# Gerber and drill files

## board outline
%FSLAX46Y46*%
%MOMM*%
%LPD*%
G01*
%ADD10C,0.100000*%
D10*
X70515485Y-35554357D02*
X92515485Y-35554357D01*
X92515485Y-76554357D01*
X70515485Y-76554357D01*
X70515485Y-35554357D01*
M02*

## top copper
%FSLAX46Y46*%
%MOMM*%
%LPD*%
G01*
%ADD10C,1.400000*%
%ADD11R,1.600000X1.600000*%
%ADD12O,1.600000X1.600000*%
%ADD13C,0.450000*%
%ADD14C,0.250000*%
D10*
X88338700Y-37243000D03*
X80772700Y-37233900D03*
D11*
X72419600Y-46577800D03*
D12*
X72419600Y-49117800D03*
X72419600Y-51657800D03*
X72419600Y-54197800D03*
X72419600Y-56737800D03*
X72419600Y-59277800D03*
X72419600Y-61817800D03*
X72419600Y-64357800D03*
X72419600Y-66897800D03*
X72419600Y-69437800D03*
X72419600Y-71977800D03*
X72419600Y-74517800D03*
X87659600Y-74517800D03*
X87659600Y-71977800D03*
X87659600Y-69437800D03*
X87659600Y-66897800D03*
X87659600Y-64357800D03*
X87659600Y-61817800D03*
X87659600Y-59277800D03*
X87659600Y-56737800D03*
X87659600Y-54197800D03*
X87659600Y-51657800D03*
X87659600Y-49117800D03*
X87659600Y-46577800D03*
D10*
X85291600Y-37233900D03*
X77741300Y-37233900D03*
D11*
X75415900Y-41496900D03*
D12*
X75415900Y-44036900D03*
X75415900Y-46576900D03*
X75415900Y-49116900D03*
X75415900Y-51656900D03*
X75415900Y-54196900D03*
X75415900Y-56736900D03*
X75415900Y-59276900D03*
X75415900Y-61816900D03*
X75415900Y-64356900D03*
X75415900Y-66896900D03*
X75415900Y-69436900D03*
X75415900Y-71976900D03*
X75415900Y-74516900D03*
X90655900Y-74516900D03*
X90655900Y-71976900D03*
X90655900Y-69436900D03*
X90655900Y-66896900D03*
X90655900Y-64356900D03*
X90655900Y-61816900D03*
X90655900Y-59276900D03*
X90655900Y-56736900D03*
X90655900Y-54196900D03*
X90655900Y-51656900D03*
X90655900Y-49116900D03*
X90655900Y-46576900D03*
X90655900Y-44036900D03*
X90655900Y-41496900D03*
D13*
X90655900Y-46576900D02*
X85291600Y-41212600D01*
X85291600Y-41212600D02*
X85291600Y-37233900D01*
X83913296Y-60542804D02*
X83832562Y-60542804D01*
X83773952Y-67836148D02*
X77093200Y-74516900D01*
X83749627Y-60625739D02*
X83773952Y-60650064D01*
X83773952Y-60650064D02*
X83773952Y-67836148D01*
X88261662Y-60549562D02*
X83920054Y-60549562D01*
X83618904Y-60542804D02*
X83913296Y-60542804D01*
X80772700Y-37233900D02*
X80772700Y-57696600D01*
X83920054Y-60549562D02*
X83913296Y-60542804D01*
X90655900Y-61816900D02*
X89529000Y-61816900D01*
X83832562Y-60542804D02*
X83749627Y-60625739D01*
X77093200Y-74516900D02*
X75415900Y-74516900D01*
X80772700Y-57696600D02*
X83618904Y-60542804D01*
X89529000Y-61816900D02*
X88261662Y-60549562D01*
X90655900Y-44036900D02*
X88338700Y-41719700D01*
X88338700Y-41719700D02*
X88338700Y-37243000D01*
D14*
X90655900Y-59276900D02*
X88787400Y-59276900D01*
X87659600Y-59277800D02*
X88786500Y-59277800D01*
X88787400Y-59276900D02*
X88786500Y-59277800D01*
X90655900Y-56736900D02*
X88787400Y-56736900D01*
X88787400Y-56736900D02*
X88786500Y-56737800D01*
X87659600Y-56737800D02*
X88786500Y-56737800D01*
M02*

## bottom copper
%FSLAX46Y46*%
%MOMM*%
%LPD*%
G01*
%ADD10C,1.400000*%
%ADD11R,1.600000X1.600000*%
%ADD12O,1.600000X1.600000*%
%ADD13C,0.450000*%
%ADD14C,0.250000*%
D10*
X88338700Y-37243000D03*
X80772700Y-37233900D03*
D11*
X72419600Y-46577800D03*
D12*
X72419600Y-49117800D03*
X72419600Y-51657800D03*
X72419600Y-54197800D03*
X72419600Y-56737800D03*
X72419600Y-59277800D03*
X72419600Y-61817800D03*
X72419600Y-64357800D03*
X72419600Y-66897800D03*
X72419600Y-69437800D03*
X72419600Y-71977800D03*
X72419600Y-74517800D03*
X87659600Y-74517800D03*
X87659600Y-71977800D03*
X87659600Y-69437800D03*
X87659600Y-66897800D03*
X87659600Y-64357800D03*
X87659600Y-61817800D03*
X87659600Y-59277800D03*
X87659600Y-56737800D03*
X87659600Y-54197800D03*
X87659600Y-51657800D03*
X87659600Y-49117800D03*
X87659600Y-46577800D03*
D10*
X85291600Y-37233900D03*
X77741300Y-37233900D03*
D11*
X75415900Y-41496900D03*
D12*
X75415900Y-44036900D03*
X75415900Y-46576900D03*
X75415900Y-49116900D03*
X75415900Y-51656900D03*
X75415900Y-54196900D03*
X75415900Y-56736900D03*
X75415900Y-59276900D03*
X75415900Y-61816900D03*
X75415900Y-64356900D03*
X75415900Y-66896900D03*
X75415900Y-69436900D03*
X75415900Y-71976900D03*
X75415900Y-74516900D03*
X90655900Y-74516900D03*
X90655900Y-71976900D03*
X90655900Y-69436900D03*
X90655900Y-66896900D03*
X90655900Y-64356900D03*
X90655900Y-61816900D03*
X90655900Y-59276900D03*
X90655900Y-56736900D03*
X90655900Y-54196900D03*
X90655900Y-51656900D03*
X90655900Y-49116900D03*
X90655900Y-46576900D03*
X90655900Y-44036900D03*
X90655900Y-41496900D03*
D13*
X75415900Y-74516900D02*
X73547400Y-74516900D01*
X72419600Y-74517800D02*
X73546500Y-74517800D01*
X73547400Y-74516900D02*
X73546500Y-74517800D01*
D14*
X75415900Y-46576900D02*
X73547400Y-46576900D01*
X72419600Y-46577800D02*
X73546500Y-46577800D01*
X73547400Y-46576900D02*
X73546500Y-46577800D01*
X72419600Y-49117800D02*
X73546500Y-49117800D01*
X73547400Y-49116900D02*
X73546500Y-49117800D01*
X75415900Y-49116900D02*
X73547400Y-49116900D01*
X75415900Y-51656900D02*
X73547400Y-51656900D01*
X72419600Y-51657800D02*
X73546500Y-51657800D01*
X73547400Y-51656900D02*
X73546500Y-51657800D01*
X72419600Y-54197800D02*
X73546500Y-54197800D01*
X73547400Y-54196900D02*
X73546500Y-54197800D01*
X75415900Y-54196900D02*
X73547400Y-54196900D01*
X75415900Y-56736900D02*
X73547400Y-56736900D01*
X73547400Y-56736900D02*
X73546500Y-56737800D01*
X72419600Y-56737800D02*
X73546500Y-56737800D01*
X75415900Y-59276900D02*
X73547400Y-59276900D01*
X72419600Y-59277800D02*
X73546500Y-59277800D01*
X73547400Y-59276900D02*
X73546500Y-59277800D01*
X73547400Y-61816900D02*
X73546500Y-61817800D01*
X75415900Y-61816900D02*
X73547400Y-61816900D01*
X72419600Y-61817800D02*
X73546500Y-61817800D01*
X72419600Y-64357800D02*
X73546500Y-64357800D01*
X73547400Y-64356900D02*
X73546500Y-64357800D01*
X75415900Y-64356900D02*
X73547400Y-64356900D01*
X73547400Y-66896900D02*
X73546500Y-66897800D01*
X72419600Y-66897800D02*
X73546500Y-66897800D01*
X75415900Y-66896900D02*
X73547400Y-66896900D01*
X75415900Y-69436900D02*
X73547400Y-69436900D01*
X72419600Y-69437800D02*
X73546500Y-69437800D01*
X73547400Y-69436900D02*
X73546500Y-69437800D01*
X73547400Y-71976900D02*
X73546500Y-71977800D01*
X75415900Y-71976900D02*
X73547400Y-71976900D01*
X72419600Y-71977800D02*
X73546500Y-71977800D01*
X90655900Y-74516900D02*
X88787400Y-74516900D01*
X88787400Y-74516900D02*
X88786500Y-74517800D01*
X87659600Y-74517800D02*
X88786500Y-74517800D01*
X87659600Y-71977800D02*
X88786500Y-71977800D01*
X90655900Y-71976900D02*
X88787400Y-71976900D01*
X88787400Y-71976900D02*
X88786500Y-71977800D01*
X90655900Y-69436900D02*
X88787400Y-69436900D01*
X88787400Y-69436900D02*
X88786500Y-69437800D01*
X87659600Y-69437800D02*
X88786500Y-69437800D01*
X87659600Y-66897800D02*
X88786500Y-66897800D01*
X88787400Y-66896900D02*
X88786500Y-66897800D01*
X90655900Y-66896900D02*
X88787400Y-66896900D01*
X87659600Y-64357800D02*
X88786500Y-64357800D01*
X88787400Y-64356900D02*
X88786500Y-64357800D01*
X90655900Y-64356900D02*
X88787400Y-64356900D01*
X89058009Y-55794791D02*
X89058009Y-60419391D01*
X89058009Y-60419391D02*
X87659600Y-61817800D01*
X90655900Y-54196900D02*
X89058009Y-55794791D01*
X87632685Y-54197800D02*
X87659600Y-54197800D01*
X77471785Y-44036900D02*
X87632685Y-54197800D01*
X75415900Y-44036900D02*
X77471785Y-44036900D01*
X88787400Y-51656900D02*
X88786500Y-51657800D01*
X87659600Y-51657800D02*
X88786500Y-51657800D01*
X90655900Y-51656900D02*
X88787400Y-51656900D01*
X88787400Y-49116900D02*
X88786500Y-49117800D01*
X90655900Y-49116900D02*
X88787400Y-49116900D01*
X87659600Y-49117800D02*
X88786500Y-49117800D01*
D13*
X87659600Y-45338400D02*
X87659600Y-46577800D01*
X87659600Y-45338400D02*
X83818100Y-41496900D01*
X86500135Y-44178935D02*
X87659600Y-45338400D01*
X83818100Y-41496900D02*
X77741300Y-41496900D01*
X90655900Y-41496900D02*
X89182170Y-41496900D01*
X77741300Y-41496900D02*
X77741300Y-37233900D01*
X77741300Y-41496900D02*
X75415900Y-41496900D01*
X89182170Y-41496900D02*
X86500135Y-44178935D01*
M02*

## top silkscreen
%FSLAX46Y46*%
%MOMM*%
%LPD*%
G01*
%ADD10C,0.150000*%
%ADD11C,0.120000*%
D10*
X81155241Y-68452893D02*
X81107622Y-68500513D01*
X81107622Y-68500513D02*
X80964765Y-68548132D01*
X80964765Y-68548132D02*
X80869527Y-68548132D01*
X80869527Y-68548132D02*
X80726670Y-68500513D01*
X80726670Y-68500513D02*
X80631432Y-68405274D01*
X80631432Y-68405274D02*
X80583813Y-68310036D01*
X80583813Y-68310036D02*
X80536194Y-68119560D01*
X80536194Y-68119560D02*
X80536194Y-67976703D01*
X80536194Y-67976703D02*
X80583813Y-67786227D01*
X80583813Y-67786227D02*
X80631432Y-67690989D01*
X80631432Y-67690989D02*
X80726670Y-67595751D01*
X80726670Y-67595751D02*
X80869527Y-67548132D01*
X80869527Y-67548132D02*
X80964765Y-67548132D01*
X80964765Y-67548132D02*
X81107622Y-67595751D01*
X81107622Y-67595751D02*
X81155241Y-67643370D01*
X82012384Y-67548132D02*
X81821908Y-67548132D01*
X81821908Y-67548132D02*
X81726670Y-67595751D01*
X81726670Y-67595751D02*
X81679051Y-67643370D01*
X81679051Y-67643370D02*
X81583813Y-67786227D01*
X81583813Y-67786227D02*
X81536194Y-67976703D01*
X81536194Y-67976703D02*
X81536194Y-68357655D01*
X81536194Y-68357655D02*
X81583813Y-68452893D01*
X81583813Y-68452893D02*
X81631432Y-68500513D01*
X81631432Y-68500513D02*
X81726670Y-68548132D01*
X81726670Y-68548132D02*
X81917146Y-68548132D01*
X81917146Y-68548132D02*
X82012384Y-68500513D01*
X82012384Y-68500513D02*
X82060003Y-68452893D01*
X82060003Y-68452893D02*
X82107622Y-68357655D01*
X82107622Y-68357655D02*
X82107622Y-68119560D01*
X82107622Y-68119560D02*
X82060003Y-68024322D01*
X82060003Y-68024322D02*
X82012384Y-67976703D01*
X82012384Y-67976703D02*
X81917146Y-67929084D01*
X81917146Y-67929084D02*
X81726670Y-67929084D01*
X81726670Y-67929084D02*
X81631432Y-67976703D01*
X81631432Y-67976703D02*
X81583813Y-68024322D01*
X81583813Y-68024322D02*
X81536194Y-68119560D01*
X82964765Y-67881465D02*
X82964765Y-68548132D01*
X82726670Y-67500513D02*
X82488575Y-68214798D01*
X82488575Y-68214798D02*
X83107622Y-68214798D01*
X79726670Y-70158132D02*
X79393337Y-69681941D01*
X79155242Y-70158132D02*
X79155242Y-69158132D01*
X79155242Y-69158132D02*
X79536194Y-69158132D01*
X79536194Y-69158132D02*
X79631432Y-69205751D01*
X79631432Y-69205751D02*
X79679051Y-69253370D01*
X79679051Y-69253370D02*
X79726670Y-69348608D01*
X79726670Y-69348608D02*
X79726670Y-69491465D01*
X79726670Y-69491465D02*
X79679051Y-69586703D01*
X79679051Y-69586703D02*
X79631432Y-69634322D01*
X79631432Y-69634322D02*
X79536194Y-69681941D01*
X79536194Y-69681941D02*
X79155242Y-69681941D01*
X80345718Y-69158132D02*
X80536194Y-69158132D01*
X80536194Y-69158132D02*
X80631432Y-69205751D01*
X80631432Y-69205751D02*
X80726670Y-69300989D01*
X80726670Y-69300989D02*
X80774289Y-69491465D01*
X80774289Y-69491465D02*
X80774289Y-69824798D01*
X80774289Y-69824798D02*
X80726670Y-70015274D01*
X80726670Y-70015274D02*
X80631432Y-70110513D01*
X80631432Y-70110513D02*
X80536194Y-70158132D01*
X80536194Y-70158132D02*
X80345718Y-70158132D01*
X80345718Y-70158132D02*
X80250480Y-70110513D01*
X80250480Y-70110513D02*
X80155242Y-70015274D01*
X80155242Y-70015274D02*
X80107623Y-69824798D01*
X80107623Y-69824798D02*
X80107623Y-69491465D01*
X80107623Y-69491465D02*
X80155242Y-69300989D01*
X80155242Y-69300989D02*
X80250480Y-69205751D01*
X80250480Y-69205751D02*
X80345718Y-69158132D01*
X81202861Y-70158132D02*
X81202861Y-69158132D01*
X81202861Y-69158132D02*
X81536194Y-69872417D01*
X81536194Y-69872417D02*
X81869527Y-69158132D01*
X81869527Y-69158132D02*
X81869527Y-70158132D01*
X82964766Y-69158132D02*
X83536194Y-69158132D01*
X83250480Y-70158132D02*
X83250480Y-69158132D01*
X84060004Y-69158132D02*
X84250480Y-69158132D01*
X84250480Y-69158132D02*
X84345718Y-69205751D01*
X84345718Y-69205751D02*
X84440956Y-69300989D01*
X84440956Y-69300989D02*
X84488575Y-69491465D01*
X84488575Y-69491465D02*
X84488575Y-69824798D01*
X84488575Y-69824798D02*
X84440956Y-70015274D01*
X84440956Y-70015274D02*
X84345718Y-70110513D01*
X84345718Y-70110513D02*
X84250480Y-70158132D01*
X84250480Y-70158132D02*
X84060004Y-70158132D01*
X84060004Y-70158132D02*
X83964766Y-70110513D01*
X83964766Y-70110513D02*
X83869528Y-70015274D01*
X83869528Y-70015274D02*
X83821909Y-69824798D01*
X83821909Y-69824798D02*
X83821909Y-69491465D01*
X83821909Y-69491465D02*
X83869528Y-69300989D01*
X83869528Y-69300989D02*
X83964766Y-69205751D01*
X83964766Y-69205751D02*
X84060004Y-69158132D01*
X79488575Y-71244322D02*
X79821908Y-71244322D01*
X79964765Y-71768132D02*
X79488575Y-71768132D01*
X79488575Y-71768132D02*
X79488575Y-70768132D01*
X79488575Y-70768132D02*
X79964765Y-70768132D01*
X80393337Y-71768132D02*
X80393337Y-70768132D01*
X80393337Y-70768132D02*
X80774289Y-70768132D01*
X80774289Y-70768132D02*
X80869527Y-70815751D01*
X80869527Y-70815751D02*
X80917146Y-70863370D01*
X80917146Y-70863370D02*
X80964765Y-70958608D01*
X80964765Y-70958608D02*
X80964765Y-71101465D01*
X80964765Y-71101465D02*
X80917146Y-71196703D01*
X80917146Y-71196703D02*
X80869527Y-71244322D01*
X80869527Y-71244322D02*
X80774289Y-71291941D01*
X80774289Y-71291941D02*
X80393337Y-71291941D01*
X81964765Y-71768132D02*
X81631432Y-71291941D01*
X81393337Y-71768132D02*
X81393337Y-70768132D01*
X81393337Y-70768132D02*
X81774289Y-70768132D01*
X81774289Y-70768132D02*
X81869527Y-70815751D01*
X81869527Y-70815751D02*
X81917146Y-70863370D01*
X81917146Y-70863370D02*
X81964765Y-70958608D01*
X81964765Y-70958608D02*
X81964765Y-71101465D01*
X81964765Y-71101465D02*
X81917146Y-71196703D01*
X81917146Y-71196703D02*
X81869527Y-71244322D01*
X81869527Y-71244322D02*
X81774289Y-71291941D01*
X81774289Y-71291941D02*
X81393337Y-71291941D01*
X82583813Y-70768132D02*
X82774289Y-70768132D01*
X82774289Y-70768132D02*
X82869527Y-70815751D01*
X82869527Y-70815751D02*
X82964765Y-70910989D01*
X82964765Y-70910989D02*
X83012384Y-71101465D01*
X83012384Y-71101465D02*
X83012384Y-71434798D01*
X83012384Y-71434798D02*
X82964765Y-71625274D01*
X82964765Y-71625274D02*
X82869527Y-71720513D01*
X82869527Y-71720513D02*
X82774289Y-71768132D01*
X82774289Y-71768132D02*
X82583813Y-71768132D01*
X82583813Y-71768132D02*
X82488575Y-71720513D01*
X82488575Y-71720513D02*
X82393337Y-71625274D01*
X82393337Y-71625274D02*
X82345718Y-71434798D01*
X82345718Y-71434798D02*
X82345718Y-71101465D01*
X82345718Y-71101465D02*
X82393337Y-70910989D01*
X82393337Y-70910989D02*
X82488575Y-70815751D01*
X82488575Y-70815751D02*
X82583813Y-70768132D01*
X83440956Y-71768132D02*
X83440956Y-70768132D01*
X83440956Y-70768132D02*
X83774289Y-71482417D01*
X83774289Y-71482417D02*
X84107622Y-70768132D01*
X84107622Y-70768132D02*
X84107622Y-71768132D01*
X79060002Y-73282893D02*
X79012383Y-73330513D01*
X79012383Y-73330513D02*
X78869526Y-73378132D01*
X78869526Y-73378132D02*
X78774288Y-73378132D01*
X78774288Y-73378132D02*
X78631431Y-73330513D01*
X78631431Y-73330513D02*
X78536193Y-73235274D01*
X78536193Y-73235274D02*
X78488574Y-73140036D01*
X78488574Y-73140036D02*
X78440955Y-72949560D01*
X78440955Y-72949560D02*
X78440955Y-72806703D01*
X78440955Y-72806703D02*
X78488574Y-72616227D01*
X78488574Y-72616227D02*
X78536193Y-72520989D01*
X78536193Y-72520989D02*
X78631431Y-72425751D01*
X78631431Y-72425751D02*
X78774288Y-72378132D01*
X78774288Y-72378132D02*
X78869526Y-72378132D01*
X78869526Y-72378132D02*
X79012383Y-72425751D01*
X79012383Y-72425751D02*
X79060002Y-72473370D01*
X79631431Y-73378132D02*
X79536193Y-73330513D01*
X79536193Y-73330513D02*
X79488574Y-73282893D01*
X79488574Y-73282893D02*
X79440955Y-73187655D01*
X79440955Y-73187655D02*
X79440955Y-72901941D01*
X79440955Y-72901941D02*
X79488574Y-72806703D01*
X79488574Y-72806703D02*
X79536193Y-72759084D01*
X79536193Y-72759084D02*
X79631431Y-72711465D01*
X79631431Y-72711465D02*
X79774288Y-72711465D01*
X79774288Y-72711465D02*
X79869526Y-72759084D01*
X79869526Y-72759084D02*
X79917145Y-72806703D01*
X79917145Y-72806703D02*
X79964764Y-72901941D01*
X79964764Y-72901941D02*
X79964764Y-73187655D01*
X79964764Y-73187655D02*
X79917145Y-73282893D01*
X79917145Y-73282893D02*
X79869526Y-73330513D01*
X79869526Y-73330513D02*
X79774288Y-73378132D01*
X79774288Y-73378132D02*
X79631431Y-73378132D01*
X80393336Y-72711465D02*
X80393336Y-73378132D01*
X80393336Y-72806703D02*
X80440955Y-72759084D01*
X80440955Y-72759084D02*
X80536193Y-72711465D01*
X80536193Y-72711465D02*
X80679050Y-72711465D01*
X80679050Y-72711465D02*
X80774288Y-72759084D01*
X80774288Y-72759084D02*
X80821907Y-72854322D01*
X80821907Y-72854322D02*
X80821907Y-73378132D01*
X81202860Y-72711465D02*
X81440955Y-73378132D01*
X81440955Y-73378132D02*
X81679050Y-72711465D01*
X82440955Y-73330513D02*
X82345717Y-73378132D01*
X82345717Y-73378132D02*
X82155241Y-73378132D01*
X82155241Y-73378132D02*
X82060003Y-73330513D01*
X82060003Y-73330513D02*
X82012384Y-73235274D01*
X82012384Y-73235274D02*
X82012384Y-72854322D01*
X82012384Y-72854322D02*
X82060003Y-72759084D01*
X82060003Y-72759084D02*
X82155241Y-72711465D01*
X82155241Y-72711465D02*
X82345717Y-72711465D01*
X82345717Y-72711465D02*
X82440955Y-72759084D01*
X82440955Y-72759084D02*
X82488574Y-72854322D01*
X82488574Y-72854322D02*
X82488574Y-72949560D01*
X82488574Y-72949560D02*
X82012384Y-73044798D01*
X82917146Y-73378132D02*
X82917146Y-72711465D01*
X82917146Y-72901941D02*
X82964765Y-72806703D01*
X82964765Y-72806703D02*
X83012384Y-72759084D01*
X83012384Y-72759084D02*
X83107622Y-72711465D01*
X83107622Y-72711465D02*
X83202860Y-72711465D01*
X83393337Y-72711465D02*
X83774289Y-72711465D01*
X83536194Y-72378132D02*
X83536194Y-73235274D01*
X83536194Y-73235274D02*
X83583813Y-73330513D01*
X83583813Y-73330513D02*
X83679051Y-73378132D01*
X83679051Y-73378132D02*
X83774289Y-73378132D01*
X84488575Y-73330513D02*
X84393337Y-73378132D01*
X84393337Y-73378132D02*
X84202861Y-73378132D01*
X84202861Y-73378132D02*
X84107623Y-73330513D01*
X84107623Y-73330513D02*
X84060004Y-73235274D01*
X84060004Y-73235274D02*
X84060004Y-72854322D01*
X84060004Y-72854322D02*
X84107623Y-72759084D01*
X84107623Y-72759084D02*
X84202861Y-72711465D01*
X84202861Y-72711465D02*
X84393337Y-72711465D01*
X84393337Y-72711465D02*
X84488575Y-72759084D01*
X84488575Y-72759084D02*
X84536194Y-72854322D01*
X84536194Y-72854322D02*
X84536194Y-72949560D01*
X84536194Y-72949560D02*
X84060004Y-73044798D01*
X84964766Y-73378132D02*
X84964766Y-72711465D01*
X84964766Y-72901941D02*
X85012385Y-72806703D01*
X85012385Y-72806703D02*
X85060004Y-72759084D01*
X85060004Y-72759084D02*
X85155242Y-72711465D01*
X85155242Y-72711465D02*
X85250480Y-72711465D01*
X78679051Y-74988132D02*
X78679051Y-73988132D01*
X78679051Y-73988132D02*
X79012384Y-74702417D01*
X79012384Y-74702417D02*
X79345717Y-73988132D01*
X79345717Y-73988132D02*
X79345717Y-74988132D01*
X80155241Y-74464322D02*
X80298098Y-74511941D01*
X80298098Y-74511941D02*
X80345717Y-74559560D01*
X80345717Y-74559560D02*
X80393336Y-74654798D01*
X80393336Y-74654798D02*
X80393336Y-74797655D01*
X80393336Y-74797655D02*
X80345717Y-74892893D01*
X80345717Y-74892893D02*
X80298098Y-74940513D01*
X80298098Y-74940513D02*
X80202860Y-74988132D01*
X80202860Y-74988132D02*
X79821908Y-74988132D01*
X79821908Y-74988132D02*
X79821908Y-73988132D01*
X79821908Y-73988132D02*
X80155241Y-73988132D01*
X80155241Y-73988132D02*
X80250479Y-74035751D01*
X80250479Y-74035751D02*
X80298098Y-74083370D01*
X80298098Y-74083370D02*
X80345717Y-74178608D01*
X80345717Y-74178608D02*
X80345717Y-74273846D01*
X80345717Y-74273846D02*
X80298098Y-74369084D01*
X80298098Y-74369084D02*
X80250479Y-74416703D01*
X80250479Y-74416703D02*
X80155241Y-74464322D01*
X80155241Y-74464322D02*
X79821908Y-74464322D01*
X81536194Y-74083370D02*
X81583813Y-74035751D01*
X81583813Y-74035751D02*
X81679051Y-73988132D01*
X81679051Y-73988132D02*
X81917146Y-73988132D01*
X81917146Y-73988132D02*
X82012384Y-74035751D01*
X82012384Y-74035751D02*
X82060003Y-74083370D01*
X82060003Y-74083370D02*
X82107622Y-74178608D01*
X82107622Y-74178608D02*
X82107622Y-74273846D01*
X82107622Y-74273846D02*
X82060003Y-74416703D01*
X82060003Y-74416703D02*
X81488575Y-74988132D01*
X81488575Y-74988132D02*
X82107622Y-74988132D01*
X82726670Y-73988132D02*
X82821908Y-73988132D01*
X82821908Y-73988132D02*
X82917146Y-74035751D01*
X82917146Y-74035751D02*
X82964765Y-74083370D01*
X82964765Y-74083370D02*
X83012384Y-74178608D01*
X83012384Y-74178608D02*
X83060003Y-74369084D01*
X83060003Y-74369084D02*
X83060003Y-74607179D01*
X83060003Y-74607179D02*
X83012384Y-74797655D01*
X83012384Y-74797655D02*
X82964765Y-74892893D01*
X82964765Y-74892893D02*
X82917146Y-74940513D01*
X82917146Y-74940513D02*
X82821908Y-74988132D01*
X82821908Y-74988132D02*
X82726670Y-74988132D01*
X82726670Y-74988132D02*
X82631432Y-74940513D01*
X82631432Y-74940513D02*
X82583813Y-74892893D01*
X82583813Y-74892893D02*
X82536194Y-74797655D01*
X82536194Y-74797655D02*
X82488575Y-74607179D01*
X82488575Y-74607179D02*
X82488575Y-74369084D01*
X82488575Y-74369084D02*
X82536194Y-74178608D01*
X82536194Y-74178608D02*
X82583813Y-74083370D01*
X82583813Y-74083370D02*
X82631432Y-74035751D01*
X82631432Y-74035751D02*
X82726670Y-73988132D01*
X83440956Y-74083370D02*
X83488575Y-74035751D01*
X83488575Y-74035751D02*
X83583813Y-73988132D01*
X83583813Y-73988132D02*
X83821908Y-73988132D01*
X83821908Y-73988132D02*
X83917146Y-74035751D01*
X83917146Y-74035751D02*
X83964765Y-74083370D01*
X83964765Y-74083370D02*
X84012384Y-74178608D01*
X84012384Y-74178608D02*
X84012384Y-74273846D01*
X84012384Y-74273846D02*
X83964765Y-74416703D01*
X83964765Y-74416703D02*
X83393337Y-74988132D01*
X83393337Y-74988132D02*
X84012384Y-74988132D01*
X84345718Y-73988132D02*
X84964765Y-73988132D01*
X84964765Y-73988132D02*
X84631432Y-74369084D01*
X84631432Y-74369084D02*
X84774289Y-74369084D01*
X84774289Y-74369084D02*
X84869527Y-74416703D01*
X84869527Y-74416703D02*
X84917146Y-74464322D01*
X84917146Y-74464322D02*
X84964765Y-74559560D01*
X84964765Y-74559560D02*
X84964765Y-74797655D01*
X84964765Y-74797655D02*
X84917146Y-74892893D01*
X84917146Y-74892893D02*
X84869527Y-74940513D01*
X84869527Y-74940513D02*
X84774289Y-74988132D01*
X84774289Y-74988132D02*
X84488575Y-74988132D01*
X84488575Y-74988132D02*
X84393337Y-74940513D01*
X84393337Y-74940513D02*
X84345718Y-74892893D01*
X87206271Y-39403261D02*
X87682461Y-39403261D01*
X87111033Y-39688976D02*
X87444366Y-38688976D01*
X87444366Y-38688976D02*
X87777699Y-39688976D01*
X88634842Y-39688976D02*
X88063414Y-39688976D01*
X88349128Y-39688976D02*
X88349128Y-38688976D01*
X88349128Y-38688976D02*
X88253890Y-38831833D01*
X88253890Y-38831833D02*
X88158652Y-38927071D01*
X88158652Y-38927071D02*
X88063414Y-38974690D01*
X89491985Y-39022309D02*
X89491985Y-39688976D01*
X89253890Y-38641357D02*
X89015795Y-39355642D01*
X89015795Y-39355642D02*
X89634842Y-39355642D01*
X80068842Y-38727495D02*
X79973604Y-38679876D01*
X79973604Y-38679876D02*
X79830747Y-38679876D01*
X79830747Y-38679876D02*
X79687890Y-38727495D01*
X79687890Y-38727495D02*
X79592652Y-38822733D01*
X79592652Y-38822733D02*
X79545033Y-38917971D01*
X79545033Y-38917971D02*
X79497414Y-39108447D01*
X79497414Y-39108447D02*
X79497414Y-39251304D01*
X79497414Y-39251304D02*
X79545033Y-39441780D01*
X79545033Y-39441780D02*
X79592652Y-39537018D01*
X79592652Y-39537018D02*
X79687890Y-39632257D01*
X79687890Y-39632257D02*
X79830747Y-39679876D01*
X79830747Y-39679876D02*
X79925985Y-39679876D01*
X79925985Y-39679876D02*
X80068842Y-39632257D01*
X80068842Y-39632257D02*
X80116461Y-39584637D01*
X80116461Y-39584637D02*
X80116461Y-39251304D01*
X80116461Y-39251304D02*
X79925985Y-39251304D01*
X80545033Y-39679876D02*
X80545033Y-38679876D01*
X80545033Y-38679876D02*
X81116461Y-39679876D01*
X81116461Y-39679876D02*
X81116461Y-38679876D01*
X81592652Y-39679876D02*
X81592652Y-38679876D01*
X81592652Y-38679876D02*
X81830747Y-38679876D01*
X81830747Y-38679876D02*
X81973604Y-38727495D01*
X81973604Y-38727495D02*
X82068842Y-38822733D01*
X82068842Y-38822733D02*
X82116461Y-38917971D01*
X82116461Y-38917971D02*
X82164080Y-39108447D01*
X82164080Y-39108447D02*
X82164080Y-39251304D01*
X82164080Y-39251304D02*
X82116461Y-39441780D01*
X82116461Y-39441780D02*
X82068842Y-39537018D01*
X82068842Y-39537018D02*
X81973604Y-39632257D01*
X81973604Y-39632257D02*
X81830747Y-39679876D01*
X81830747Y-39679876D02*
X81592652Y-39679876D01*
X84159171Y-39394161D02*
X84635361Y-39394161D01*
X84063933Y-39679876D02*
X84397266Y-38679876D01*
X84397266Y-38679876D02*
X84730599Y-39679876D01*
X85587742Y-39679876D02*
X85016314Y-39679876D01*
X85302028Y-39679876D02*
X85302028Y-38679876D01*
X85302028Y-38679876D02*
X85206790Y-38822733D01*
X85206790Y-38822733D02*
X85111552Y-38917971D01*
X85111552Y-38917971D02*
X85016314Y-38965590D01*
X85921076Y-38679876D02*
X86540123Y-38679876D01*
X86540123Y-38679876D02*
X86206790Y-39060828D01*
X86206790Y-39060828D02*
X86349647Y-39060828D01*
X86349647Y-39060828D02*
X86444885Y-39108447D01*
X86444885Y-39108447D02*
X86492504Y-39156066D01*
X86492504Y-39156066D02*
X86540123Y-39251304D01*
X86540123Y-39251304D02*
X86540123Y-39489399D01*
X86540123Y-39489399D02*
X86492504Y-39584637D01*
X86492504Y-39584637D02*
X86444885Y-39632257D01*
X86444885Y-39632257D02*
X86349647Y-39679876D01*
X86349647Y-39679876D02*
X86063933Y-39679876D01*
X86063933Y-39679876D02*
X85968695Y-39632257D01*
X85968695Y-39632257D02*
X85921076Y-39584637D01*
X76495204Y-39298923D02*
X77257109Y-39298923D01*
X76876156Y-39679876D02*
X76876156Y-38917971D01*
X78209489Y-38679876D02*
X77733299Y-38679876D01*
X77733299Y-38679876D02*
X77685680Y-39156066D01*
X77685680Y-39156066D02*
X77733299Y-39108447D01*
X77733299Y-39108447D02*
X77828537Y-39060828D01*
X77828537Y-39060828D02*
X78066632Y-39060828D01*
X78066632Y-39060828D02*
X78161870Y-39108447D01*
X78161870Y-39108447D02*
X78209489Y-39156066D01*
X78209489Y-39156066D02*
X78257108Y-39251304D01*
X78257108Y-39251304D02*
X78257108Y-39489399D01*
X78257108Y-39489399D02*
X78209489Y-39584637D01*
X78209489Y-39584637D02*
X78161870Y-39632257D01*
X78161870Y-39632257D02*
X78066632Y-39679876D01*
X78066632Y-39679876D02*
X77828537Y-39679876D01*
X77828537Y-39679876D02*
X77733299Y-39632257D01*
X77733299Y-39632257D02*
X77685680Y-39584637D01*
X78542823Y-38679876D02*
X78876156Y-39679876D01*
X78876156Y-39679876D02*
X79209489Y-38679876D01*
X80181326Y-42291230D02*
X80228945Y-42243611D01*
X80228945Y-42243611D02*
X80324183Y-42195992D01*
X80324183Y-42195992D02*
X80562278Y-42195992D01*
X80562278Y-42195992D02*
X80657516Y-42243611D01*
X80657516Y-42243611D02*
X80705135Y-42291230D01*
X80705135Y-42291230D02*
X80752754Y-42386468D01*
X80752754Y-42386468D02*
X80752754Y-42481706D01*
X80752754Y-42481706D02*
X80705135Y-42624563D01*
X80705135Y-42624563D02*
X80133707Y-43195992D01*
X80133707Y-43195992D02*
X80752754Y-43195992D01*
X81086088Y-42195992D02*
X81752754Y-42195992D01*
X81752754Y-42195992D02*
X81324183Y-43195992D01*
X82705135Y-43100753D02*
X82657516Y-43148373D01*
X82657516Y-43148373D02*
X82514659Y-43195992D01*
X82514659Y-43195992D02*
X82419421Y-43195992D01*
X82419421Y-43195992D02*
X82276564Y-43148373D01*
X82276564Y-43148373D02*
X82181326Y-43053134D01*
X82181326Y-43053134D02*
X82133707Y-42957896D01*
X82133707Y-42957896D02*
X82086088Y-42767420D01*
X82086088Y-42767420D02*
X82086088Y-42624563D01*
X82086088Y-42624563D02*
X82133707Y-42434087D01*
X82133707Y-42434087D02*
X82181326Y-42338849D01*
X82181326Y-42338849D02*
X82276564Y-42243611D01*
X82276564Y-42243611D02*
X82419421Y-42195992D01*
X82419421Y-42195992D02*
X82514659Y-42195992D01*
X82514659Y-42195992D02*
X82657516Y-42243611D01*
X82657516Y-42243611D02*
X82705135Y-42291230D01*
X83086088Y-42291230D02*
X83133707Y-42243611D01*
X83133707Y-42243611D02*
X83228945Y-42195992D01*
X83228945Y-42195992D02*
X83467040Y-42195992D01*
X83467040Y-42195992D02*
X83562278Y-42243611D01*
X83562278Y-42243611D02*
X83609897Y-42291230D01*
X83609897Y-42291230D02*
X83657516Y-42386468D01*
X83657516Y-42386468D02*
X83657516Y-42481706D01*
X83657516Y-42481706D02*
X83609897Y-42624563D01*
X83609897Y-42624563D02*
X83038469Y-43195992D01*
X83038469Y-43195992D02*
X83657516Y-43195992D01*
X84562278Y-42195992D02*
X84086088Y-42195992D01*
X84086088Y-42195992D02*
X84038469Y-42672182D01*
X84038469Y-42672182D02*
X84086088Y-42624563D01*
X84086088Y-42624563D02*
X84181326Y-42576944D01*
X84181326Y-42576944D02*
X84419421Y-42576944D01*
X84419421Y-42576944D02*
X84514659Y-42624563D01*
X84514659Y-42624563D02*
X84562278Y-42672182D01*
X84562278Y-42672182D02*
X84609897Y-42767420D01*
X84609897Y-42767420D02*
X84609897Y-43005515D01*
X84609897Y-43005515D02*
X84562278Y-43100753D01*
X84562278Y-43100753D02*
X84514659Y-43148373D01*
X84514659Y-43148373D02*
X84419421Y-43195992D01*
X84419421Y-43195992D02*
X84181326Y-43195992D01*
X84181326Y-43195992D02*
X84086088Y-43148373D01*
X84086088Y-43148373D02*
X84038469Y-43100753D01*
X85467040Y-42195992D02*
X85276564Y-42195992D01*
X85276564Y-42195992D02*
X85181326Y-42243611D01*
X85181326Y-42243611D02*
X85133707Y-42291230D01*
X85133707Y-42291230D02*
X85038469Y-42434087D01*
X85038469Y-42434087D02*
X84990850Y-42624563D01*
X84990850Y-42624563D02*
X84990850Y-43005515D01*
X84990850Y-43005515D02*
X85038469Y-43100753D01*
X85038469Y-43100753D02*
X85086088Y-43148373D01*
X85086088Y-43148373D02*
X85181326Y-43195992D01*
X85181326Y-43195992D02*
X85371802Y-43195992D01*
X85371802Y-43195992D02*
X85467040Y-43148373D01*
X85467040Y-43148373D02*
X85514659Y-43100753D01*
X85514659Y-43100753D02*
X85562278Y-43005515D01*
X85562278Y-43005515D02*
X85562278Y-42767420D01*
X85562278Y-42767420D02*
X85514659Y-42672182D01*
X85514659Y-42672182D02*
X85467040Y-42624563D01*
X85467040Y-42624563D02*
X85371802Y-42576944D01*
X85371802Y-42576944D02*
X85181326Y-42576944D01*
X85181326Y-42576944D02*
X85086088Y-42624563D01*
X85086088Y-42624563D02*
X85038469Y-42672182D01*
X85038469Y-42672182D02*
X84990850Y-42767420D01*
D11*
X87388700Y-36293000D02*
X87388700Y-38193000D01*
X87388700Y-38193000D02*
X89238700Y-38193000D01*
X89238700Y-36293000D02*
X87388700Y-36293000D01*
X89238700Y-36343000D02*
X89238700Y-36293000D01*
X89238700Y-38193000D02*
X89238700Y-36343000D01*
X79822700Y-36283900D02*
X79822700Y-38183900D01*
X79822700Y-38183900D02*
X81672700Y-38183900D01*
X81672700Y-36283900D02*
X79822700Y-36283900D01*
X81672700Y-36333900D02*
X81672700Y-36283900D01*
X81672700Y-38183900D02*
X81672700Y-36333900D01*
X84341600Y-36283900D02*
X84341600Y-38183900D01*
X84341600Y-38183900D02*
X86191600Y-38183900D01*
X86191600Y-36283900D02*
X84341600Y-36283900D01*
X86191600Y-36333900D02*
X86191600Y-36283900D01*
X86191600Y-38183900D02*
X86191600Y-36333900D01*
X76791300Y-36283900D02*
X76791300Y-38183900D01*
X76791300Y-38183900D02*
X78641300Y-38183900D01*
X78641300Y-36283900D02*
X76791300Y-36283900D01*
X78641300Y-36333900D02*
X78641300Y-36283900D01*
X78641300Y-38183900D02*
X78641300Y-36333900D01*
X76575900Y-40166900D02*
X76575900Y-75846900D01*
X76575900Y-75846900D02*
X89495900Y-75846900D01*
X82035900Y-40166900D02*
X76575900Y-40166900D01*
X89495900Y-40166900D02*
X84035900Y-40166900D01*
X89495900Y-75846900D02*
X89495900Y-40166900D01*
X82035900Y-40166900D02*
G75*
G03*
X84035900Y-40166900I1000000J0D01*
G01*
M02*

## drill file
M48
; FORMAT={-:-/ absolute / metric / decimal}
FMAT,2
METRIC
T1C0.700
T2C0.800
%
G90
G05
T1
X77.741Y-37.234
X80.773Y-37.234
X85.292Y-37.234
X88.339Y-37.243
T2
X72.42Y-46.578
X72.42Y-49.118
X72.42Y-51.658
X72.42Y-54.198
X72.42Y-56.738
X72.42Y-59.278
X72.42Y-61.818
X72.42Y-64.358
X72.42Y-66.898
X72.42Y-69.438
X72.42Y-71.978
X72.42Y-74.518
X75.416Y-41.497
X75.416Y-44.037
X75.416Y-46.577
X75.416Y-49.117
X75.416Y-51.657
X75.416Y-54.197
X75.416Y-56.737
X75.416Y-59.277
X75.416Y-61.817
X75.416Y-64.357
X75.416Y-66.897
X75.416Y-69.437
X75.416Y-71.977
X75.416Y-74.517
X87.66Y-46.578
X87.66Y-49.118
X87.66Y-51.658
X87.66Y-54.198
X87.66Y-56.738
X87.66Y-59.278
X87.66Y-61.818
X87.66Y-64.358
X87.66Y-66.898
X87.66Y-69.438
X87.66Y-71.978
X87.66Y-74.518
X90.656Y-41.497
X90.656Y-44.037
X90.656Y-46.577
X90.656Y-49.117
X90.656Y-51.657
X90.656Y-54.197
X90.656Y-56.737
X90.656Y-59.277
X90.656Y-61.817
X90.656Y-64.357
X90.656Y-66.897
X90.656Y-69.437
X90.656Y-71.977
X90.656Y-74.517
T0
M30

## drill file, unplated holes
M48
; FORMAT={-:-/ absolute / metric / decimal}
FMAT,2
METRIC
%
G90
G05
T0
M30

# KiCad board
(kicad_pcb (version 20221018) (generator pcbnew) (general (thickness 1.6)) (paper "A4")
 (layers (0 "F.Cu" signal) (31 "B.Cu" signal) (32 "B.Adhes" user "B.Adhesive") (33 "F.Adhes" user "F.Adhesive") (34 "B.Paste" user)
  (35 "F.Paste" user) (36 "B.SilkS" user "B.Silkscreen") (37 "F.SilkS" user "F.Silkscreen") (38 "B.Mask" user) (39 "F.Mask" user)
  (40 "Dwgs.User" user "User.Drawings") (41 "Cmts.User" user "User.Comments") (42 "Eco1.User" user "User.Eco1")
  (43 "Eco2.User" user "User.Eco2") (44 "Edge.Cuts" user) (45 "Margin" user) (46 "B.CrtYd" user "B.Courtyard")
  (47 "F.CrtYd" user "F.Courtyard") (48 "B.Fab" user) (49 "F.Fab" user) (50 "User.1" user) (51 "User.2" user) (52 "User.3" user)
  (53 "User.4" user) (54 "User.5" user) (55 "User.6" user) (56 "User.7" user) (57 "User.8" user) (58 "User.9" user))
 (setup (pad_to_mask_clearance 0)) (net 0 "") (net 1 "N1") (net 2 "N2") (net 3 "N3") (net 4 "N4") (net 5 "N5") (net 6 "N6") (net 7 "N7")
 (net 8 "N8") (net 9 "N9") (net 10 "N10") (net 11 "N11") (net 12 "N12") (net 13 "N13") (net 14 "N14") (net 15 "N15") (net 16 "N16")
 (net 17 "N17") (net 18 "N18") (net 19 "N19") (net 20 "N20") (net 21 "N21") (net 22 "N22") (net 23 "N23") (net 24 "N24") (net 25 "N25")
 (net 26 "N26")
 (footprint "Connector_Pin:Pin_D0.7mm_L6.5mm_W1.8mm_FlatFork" (layer "F.Cu") (at 88.3387 37.243)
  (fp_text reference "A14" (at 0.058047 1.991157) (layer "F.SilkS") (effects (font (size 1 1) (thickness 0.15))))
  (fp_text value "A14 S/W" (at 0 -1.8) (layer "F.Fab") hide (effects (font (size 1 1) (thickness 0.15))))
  (fp_line (start -0.95 -0.95) (end -0.95 0.95) (stroke (width 0.12) (type solid)) (layer "F.SilkS"))
  (fp_line (start -0.95 0.95) (end 0.9 0.95) (stroke (width 0.12) (type solid)) (layer "F.SilkS"))
  (fp_line (start 0.9 -0.95) (end -0.95 -0.95) (stroke (width 0.12) (type solid)) (layer "F.SilkS"))
  (fp_line (start 0.9 -0.9) (end 0.9 -0.95) (stroke (width 0.12) (type solid)) (layer "F.SilkS"))
  (fp_line (start 0.9 0.95) (end 0.9 -0.9) (stroke (width 0.12) (type solid)) (layer "F.SilkS"))
  (pad "1" thru_hole circle (at 0 0) (size 1.4 1.4) (drill 0.7) (layers "*.Cu" "*.Mask") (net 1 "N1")))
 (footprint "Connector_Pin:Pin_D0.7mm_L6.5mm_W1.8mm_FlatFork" (layer "F.Cu") (at 80.7727 37.2339)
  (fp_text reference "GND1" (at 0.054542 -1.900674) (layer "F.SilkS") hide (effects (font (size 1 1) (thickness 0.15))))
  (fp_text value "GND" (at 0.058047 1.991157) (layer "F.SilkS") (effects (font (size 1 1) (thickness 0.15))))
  (fp_line (start -0.95 -0.95) (end -0.95 0.95) (stroke (width 0.12) (type solid)) (layer "F.SilkS"))
  (fp_line (start -0.95 0.95) (end 0.9 0.95) (stroke (width 0.12) (type solid)) (layer "F.SilkS"))
  (fp_line (start 0.9 -0.95) (end -0.95 -0.95) (stroke (width 0.12) (type solid)) (layer "F.SilkS"))
  (fp_line (start 0.9 -0.9) (end 0.9 -0.95) (stroke (width 0.12) (type solid)) (layer "F.SilkS"))
  (fp_line (start 0.9 0.95) (end 0.9 -0.9) (stroke (width 0.12) (type solid)) (layer "F.SilkS"))
  (pad "1" thru_hole circle (at 0 0) (size 1.4 1.4) (drill 0.7) (layers "*.Cu" "*.Mask") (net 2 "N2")))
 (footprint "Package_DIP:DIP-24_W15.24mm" (layer "F.Cu") (at 72.4196 46.5778)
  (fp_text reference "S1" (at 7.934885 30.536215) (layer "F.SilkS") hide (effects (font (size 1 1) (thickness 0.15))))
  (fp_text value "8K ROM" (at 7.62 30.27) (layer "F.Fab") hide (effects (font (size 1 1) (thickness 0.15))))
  (pad "1" thru_hole rect (at 0 0) (size 1.6 1.6) (drill 0.8) (layers "*.Cu" "*.Mask") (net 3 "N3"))
  (pad "2" thru_hole oval (at 0 2.54) (size 1.6 1.6) (drill 0.8) (layers "*.Cu" "*.Mask") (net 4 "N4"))
  (pad "3" thru_hole oval (at 0 5.08) (size 1.6 1.6) (drill 0.8) (layers "*.Cu" "*.Mask") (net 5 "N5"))
  (pad "4" thru_hole oval (at 0 7.62) (size 1.6 1.6) (drill 0.8) (layers "*.Cu" "*.Mask") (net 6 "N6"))
  (pad "5" thru_hole oval (at 0 10.16) (size 1.6 1.6) (drill 0.8) (layers "*.Cu" "*.Mask") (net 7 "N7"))
  (pad "6" thru_hole oval (at 0 12.7) (size 1.6 1.6) (drill 0.8) (layers "*.Cu" "*.Mask") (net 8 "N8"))
  (pad "7" thru_hole oval (at 0 15.24) (size 1.6 1.6) (drill 0.8) (layers "*.Cu" "*.Mask") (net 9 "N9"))
  (pad "8" thru_hole oval (at 0 17.78) (size 1.6 1.6) (drill 0.8) (layers "*.Cu" "*.Mask") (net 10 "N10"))
  (pad "9" thru_hole oval (at 0 20.32) (size 1.6 1.6) (drill 0.8) (layers "*.Cu" "*.Mask") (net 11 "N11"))
  (pad "10" thru_hole oval (at 0 22.86) (size 1.6 1.6) (drill 0.8) (layers "*.Cu" "*.Mask") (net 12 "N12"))
  (pad "11" thru_hole oval (at 0 25.4) (size 1.6 1.6) (drill 0.8) (layers "*.Cu" "*.Mask") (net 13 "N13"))
  (pad "12" thru_hole oval (at 0 27.94) (size 1.6 1.6) (drill 0.8) (layers "*.Cu" "*.Mask") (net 2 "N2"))
  (pad "13" thru_hole oval (at 15.24 27.94) (size 1.6 1.6) (drill 0.8) (layers "*.Cu" "*.Mask") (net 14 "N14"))
  (pad "14" thru_hole oval (at 15.24 25.4) (size 1.6 1.6) (drill 0.8) (layers "*.Cu" "*.Mask") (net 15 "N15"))
  (pad "15" thru_hole oval (at 15.24 22.86) (size 1.6 1.6) (drill 0.8) (layers "*.Cu" "*.Mask") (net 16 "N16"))
  (pad "16" thru_hole oval (at 15.24 20.32) (size 1.6 1.6) (drill 0.8) (layers "*.Cu" "*.Mask") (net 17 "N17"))
  (pad "17" thru_hole oval (at 15.24 17.78) (size 1.6 1.6) (drill 0.8) (layers "*.Cu" "*.Mask") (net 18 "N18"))
  (pad "18" thru_hole oval (at 15.24 15.24) (size 1.6 1.6) (drill 0.8) (layers "*.Cu" "*.Mask") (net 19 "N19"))
  (pad "19" thru_hole oval (at 15.24 12.7) (size 1.6 1.6) (drill 0.8) (layers "*.Cu" "*.Mask") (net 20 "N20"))
  (pad "20" thru_hole oval (at 15.24 10.16) (size 1.6 1.6) (drill 0.8) (layers "*.Cu" "*.Mask") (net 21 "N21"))
  (pad "21" thru_hole oval (at 15.24 7.62) (size 1.6 1.6) (drill 0.8) (layers "*.Cu" "*.Mask") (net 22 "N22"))
  (pad "22" thru_hole oval (at 15.24 5.08) (size 1.6 1.6) (drill 0.8) (layers "*.Cu" "*.Mask") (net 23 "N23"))
  (pad "23" thru_hole oval (at 15.24 2.54) (size 1.6 1.6) (drill 0.8) (layers "*.Cu" "*.Mask") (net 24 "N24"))
  (pad "24" thru_hole oval (at 15.24 0) (size 1.6 1.6) (drill 0.8) (layers "*.Cu" "*.Mask") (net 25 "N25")))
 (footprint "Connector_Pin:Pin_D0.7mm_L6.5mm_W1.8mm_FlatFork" (layer "F.Cu") (at 85.2916 37.2339)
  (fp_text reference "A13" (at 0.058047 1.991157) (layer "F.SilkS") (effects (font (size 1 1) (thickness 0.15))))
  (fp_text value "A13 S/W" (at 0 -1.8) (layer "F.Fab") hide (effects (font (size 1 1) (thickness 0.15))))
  (fp_line (start -0.95 -0.95) (end -0.95 0.95) (stroke (width 0.12) (type solid)) (layer "F.SilkS"))
  (fp_line (start -0.95 0.95) (end 0.9 0.95) (stroke (width 0.12) (type solid)) (layer "F.SilkS"))
  (fp_line (start 0.9 -0.95) (end -0.95 -0.95) (stroke (width 0.12) (type solid)) (layer "F.SilkS"))
  (fp_line (start 0.9 -0.9) (end 0.9 -0.95) (stroke (width 0.12) (type solid)) (layer "F.SilkS"))
  (fp_line (start 0.9 0.95) (end 0.9 -0.9) (stroke (width 0.12) (type solid)) (layer "F.SilkS"))
  (pad "1" thru_hole circle (at 0 0) (size 1.4 1.4) (drill 0.7) (layers "*.Cu" "*.Mask") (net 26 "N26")))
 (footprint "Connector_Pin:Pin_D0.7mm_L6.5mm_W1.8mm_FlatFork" (layer "F.Cu") (at 77.7413 37.2339)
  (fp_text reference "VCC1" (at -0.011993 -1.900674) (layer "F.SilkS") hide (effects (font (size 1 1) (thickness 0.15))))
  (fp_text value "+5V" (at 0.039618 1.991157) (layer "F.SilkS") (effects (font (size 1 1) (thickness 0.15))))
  (fp_line (start -0.95 -0.95) (end -0.95 0.95) (stroke (width 0.12) (type solid)) (layer "F.SilkS"))
  (fp_line (start -0.95 0.95) (end 0.9 0.95) (stroke (width 0.12) (type solid)) (layer "F.SilkS"))
  (fp_line (start 0.9 -0.95) (end -0.95 -0.95) (stroke (width 0.12) (type solid)) (layer "F.SilkS"))
  (fp_line (start 0.9 -0.9) (end 0.9 -0.95) (stroke (width 0.12) (type solid)) (layer "F.SilkS"))
  (fp_line (start 0.9 0.95) (end 0.9 -0.9) (stroke (width 0.12) (type solid)) (layer "F.SilkS"))
  (pad "1" thru_hole circle (at 0 0) (size 1.4 1.4) (drill 0.7) (layers "*.Cu" "*.Mask") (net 25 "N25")))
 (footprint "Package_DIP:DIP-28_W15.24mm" (layer "F.Cu") (at 75.4159 41.4969)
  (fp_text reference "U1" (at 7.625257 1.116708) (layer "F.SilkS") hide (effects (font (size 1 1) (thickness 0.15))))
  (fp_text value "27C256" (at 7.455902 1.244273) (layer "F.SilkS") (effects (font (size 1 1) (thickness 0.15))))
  (fp_line (start 1.16 -1.33) (end 1.16 34.35) (stroke (width 0.12) (type solid)) (layer "F.SilkS"))
  (fp_line (start 1.16 34.35) (end 14.08 34.35) (stroke (width 0.12) (type solid)) (layer "F.SilkS"))
  (fp_line (start 6.62 -1.33) (end 1.16 -1.33) (stroke (width 0.12) (type solid)) (layer "F.SilkS"))
  (fp_line (start 14.08 -1.33) (end 8.62 -1.33) (stroke (width 0.12) (type solid)) (layer "F.SilkS"))
  (fp_line (start 14.08 34.35) (end 14.08 -1.33) (stroke (width 0.12) (type solid)) (layer "F.SilkS"))
  (fp_arc (start 8.62 -1.33) (mid 7.62 -0.33) (end 6.62 -1.33) (stroke (width 0.12) (type solid)) (layer "F.SilkS"))
  (pad "1" thru_hole rect (at 0 0) (size 1.6 1.6) (drill 0.8) (layers "*.Cu" "*.Mask") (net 25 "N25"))
  (pad "2" thru_hole oval (at 0 2.54) (size 1.6 1.6) (drill 0.8) (layers "*.Cu" "*.Mask") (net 22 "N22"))
  (pad "3" thru_hole oval (at 0 5.08) (size 1.6 1.6) (drill 0.8) (layers "*.Cu" "*.Mask") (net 3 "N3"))
  (pad "4" thru_hole oval (at 0 7.62) (size 1.6 1.6) (drill 0.8) (layers "*.Cu" "*.Mask") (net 4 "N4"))
  (pad "5" thru_hole oval (at 0 10.16) (size 1.6 1.6) (drill 0.8) (layers "*.Cu" "*.Mask") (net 5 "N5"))
  (pad "6" thru_hole oval (at 0 12.7) (size 1.6 1.6) (drill 0.8) (layers "*.Cu" "*.Mask") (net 6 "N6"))
  (pad "7" thru_hole oval (at 0 15.24) (size 1.6 1.6) (drill 0.8) (layers "*.Cu" "*.Mask") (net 7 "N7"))
  (pad "8" thru_hole oval (at 0 17.78) (size 1.6 1.6) (drill 0.8) (layers "*.Cu" "*.Mask") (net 8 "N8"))
  (pad "9" thru_hole oval (at 0 20.32) (size 1.6 1.6) (drill 0.8) (layers "*.Cu" "*.Mask") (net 9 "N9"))
  (pad "10" thru_hole oval (at 0 22.86) (size 1.6 1.6) (drill 0.8) (layers "*.Cu" "*.Mask") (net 10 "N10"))
  (pad "11" thru_hole oval (at 0 25.4) (size 1.6 1.6) (drill 0.8) (layers "*.Cu" "*.Mask") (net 11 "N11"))
  (pad "12" thru_hole oval (at 0 27.94) (size 1.6 1.6) (drill 0.8) (layers "*.Cu" "*.Mask") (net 12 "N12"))
  (pad "13" thru_hole oval (at 0 30.48) (size 1.6 1.6) (drill 0.8) (layers "*.Cu" "*.Mask") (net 13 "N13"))
  (pad "14" thru_hole oval (at 0 33.02) (size 1.6 1.6) (drill 0.8) (layers "*.Cu" "*.Mask") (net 2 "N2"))
  (pad "15" thru_hole oval (at 15.24 33.02) (size 1.6 1.6) (drill 0.8) (layers "*.Cu" "*.Mask") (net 14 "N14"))
  (pad "16" thru_hole oval (at 15.24 30.48) (size 1.6 1.6) (drill 0.8) (layers "*.Cu" "*.Mask") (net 15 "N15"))
  (pad "17" thru_hole oval (at 15.24 27.94) (size 1.6 1.6) (drill 0.8) (layers "*.Cu" "*.Mask") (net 16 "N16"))
  (pad "18" thru_hole oval (at 15.24 25.4) (size 1.6 1.6) (drill 0.8) (layers "*.Cu" "*.Mask") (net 17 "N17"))
  (pad "19" thru_hole oval (at 15.24 22.86) (size 1.6 1.6) (drill 0.8) (layers "*.Cu" "*.Mask") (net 18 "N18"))
  (pad "20" thru_hole oval (at 15.24 20.32) (size 1.6 1.6) (drill 0.8) (layers "*.Cu" "*.Mask") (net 2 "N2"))
  (pad "21" thru_hole oval (at 15.24 17.78) (size 1.6 1.6) (drill 0.8) (layers "*.Cu" "*.Mask") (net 20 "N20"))
  (pad "22" thru_hole oval (at 15.24 15.24) (size 1.6 1.6) (drill 0.8) (layers "*.Cu" "*.Mask") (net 21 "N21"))
  (pad "23" thru_hole oval (at 15.24 12.7) (size 1.6 1.6) (drill 0.8) (layers "*.Cu" "*.Mask") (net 19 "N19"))
  (pad "24" thru_hole oval (at 15.24 10.16) (size 1.6 1.6) (drill 0.8) (layers "*.Cu" "*.Mask") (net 23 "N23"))
  (pad "25" thru_hole oval (at 15.24 7.62) (size 1.6 1.6) (drill 0.8) (layers "*.Cu" "*.Mask") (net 24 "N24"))
  (pad "26" thru_hole oval (at 15.24 5.08) (size 1.6 1.6) (drill 0.8) (layers "*.Cu" "*.Mask") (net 26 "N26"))
  (pad "27" thru_hole oval (at 15.24 2.54) (size 1.6 1.6) (drill 0.8) (layers "*.Cu" "*.Mask") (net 1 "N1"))
  (pad "28" thru_hole oval (at 15.24 0) (size 1.6 1.6) (drill 0.8) (layers "*.Cu" "*.Mask") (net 25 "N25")))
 (gr_rect (start 70.515485 35.554357) (end 92.515485 76.554357) (stroke (width 0.1) (type default)) (fill none) (layer "Edge.Cuts"))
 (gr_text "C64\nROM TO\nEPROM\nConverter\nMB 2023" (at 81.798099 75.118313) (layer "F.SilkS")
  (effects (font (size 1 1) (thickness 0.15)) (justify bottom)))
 (segment (start 90.6559 46.5769) (end 85.2916 41.2126) (width 0.45) (layer "F.Cu") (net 26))
 (segment (start 85.2916 41.2126) (end 85.2916 37.2339) (width 0.45) (layer "F.Cu") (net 26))
 (segment (start 83.913296 60.542804) (end 83.832562 60.542804) (width 0.45) (layer "F.Cu") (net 2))
 (segment (start 83.773952 67.836148) (end 77.0932 74.5169) (width 0.45) (layer "F.Cu") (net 2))
 (segment (start 83.749627 60.625739) (end 83.773952 60.650064) (width 0.45) (layer "F.Cu") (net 2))
 (segment (start 83.773952 60.650064) (end 83.773952 67.836148) (width 0.45) (layer "F.Cu") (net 2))
 (segment (start 88.261662 60.549562) (end 83.920054 60.549562) (width 0.45) (layer "F.Cu") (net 2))
 (segment (start 83.618904 60.542804) (end 83.913296 60.542804) (width 0.45) (layer "F.Cu") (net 2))
 (segment (start 80.7727 37.2339) (end 80.7727 57.6966) (width 0.45) (layer "F.Cu") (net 2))
 (segment (start 83.920054 60.549562) (end 83.913296 60.542804) (width 0.45) (layer "F.Cu") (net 2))
 (segment (start 90.6559 61.8169) (end 89.529 61.8169) (width 0.45) (layer "F.Cu") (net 2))
 (segment (start 83.832562 60.542804) (end 83.749627 60.625739) (width 0.45) (layer "F.Cu") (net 2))
 (segment (start 77.0932 74.5169) (end 75.4159 74.5169) (width 0.45) (layer "F.Cu") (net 2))
 (segment (start 80.7727 57.6966) (end 83.618904 60.542804) (width 0.45) (layer "F.Cu") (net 2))
 (segment (start 89.529 61.8169) (end 88.261662 60.549562) (width 0.45) (layer "F.Cu") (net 2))
 (segment (start 75.4159 74.5169) (end 73.5474 74.5169) (width 0.45) (layer "B.Cu") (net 2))
 (segment (start 72.4196 74.5178) (end 73.5465 74.5178) (width 0.45) (layer "B.Cu") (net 2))
 (segment (start 73.5474 74.5169) (end 73.5465 74.5178) (width 0.45) (layer "B.Cu") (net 2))
 (segment (start 90.6559 44.0369) (end 88.3387 41.7197) (width 0.45) (layer "F.Cu") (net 1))
 (segment (start 88.3387 41.7197) (end 88.3387 37.243) (width 0.45) (layer "F.Cu") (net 1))
 (segment (start 75.4159 46.5769) (end 73.5474 46.5769) (width 0.25) (layer "B.Cu") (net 3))
 (segment (start 72.4196 46.5778) (end 73.5465 46.5778) (width 0.25) (layer "B.Cu") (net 3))
 (segment (start 73.5474 46.5769) (end 73.5465 46.5778) (width 0.25) (layer "B.Cu") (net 3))
 (segment (start 72.4196 49.1178) (end 73.5465 49.1178) (width 0.25) (layer "B.Cu") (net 4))
 (segment (start 73.5474 49.1169) (end 73.5465 49.1178) (width 0.25) (layer "B.Cu") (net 4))
 (segment (start 75.4159 49.1169) (end 73.5474 49.1169) (width 0.25) (layer "B.Cu") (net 4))
 (segment (start 75.4159 51.6569) (end 73.5474 51.6569) (width 0.25) (layer "B.Cu") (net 5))
 (segment (start 72.4196 51.6578) (end 73.5465 51.6578) (width 0.25) (layer "B.Cu") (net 5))
 (segment (start 73.5474 51.6569) (end 73.5465 51.6578) (width 0.25) (layer "B.Cu") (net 5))
 (segment (start 72.4196 54.1978) (end 73.5465 54.1978) (width 0.25) (layer "B.Cu") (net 6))
 (segment (start 73.5474 54.1969) (end 73.5465 54.1978) (width 0.25) (layer "B.Cu") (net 6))
 (segment (start 75.4159 54.1969) (end 73.5474 54.1969) (width 0.25) (layer "B.Cu") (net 6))
 (segment (start 75.4159 56.7369) (end 73.5474 56.7369) (width 0.25) (layer "B.Cu") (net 7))
 (segment (start 73.5474 56.7369) (end 73.5465 56.7378) (width 0.25) (layer "B.Cu") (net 7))
 (segment (start 72.4196 56.7378) (end 73.5465 56.7378) (width 0.25) (layer "B.Cu") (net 7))
 (segment (start 75.4159 59.2769) (end 73.5474 59.2769) (width 0.25) (layer "B.Cu") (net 8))
 (segment (start 72.4196 59.2778) (end 73.5465 59.2778) (width 0.25) (layer "B.Cu") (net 8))
 (segment (start 73.5474 59.2769) (end 73.5465 59.2778) (width 0.25) (layer "B.Cu") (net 8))
 (segment (start 73.5474 61.8169) (end 73.5465 61.8178) (width 0.25) (layer "B.Cu") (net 9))
 (segment (start 75.4159 61.8169) (end 73.5474 61.8169) (width 0.25) (layer "B.Cu") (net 9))
 (segment (start 72.4196 61.8178) (end 73.5465 61.8178) (width 0.25) (layer "B.Cu") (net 9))
 (segment (start 72.4196 64.3578) (end 73.5465 64.3578) (width 0.25) (layer "B.Cu") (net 10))
 (segment (start 73.5474 64.3569) (end 73.5465 64.3578) (width 0.25) (layer "B.Cu") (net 10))
 (segment (start 75.4159 64.3569) (end 73.5474 64.3569) (width 0.25) (layer "B.Cu") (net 10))
 (segment (start 73.5474 66.8969) (end 73.5465 66.8978) (width 0.25) (layer "B.Cu") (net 11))
 (segment (start 72.4196 66.8978) (end 73.5465 66.8978) (width 0.25) (layer "B.Cu") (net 11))
 (segment (start 75.4159 66.8969) (end 73.5474 66.8969) (width 0.25) (layer "B.Cu") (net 11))
 (segment (start 75.4159 69.4369) (end 73.5474 69.4369) (width 0.25) (layer "B.Cu") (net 12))
 (segment (start 72.4196 69.4378) (end 73.5465 69.4378) (width 0.25) (layer "B.Cu") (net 12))
 (segment (start 73.5474 69.4369) (end 73.5465 69.4378) (width 0.25) (layer "B.Cu") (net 12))
 (segment (start 73.5474 71.9769) (end 73.5465 71.9778) (width 0.25) (layer "B.Cu") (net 13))
 (segment (start 75.4159 71.9769) (end 73.5474 71.9769) (width 0.25) (layer "B.Cu") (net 13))
 (segment (start 72.4196 71.9778) (end 73.5465 71.9778) (width 0.25) (layer "B.Cu") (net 13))
 (segment (start 90.6559 74.5169) (end 88.7874 74.5169) (width 0.25) (layer "B.Cu") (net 14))
 (segment (start 88.7874 74.5169) (end 88.7865 74.5178) (width 0.25) (layer "B.Cu") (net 14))
 (segment (start 87.6596 74.5178) (end 88.7865 74.5178) (width 0.25) (layer "B.Cu") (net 14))
 (segment (start 87.6596 71.9778) (end 88.7865 71.9778) (width 0.25) (layer "B.Cu") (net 15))
 (segment (start 90.6559 71.9769) (end 88.7874 71.9769) (width 0.25) (layer "B.Cu") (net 15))
 (segment (start 88.7874 71.9769) (end 88.7865 71.9778) (width 0.25) (layer "B.Cu") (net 15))
 (segment (start 90.6559 69.4369) (end 88.7874 69.4369) (width 0.25) (layer "B.Cu") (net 16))
 (segment (start 88.7874 69.4369) (end 88.7865 69.4378) (width 0.25) (layer "B.Cu") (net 16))
 (segment (start 87.6596 69.4378) (end 88.7865 69.4378) (width 0.25) (layer "B.Cu") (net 16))
 (segment (start 87.6596 66.8978) (end 88.7865 66.8978) (width 0.25) (layer "B.Cu") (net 17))
 (segment (start 88.7874 66.8969) (end 88.7865 66.8978) (width 0.25) (layer "B.Cu") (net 17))
 (segment (start 90.6559 66.8969) (end 88.7874 66.8969) (width 0.25) (layer "B.Cu") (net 17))
 (segment (start 87.6596 64.3578) (end 88.7865 64.3578) (width 0.25) (layer "B.Cu") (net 18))
 (segment (start 88.7874 64.3569) (end 88.7865 64.3578) (width 0.25) (layer "B.Cu") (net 18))
 (segment (start 90.6559 64.3569) (end 88.7874 64.3569) (width 0.25) (layer "B.Cu") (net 18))
 (segment (start 89.058009 55.794791) (end 89.058009 60.419391) (width 0.25) (layer "B.Cu") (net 19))
 (segment (start 89.058009 60.419391) (end 87.6596 61.8178) (width 0.25) (layer "B.Cu") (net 19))
 (segment (start 90.6559 54.1969) (end 89.058009 55.794791) (width 0.25) (layer "B.Cu") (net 19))
 (segment (start 90.6559 59.2769) (end 88.7874 59.2769) (width 0.25) (layer "F.Cu") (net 20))
 (segment (start 87.6596 59.2778) (end 88.7865 59.2778) (width 0.25) (layer "F.Cu") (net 20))
 (segment (start 88.7874 59.2769) (end 88.7865 59.2778) (width 0.25) (layer "F.Cu") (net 20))
 (segment (start 90.6559 56.7369) (end 88.7874 56.7369) (width 0.25) (layer "F.Cu") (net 21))
 (segment (start 88.7874 56.7369) (end 88.7865 56.7378) (width 0.25) (layer "F.Cu") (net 21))
 (segment (start 87.6596 56.7378) (end 88.7865 56.7378) (width 0.25) (layer "F.Cu") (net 21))
 (segment (start 87.632685 54.1978) (end 87.6596 54.1978) (width 0.25) (layer "B.Cu") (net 22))
 (segment (start 77.471785 44.0369) (end 87.632685 54.1978) (width 0.25) (layer "B.Cu") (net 22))
 (segment (start 75.4159 44.0369) (end 77.471785 44.0369) (width 0.25) (layer "B.Cu") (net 22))
 (segment (start 88.7874 51.6569) (end 88.7865 51.6578) (width 0.25) (layer "B.Cu") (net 23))
 (segment (start 87.6596 51.6578) (end 88.7865 51.6578) (width 0.25) (layer "B.Cu") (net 23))
 (segment (start 90.6559 51.6569) (end 88.7874 51.6569) (width 0.25) (layer "B.Cu") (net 23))
 (segment (start 88.7874 49.1169) (end 88.7865 49.1178) (width 0.25) (layer "B.Cu") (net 24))
 (segment (start 90.6559 49.1169) (end 88.7874 49.1169) (width 0.25) (layer "B.Cu") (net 24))
 (segment (start 87.6596 49.1178) (end 88.7865 49.1178) (width 0.25) (layer "B.Cu") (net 24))
 (segment (start 87.6596 45.3384) (end 87.6596 46.5778) (width 0.45) (layer "B.Cu") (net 25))
 (segment (start 87.6596 45.3384) (end 83.8181 41.4969) (width 0.45) (layer "B.Cu") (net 25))
 (segment (start 86.500135 44.178935) (end 87.6596 45.3384) (width 0.45) (layer "B.Cu") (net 25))
 (segment (start 83.8181 41.4969) (end 77.7413 41.4969) (width 0.45) (layer "B.Cu") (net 25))
 (segment (start 90.6559 41.4969) (end 89.18217 41.4969) (width 0.45) (layer "B.Cu") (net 25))
 (segment (start 77.7413 41.4969) (end 77.7413 37.2339) (width 0.45) (layer "B.Cu") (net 25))
 (segment (start 77.7413 41.4969) (end 75.4159 41.4969) (width 0.45) (layer "B.Cu") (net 25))
 (segment (start 89.18217 41.4969) (end 86.500135 44.178935) (width 0.45) (layer "B.Cu") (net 25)))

